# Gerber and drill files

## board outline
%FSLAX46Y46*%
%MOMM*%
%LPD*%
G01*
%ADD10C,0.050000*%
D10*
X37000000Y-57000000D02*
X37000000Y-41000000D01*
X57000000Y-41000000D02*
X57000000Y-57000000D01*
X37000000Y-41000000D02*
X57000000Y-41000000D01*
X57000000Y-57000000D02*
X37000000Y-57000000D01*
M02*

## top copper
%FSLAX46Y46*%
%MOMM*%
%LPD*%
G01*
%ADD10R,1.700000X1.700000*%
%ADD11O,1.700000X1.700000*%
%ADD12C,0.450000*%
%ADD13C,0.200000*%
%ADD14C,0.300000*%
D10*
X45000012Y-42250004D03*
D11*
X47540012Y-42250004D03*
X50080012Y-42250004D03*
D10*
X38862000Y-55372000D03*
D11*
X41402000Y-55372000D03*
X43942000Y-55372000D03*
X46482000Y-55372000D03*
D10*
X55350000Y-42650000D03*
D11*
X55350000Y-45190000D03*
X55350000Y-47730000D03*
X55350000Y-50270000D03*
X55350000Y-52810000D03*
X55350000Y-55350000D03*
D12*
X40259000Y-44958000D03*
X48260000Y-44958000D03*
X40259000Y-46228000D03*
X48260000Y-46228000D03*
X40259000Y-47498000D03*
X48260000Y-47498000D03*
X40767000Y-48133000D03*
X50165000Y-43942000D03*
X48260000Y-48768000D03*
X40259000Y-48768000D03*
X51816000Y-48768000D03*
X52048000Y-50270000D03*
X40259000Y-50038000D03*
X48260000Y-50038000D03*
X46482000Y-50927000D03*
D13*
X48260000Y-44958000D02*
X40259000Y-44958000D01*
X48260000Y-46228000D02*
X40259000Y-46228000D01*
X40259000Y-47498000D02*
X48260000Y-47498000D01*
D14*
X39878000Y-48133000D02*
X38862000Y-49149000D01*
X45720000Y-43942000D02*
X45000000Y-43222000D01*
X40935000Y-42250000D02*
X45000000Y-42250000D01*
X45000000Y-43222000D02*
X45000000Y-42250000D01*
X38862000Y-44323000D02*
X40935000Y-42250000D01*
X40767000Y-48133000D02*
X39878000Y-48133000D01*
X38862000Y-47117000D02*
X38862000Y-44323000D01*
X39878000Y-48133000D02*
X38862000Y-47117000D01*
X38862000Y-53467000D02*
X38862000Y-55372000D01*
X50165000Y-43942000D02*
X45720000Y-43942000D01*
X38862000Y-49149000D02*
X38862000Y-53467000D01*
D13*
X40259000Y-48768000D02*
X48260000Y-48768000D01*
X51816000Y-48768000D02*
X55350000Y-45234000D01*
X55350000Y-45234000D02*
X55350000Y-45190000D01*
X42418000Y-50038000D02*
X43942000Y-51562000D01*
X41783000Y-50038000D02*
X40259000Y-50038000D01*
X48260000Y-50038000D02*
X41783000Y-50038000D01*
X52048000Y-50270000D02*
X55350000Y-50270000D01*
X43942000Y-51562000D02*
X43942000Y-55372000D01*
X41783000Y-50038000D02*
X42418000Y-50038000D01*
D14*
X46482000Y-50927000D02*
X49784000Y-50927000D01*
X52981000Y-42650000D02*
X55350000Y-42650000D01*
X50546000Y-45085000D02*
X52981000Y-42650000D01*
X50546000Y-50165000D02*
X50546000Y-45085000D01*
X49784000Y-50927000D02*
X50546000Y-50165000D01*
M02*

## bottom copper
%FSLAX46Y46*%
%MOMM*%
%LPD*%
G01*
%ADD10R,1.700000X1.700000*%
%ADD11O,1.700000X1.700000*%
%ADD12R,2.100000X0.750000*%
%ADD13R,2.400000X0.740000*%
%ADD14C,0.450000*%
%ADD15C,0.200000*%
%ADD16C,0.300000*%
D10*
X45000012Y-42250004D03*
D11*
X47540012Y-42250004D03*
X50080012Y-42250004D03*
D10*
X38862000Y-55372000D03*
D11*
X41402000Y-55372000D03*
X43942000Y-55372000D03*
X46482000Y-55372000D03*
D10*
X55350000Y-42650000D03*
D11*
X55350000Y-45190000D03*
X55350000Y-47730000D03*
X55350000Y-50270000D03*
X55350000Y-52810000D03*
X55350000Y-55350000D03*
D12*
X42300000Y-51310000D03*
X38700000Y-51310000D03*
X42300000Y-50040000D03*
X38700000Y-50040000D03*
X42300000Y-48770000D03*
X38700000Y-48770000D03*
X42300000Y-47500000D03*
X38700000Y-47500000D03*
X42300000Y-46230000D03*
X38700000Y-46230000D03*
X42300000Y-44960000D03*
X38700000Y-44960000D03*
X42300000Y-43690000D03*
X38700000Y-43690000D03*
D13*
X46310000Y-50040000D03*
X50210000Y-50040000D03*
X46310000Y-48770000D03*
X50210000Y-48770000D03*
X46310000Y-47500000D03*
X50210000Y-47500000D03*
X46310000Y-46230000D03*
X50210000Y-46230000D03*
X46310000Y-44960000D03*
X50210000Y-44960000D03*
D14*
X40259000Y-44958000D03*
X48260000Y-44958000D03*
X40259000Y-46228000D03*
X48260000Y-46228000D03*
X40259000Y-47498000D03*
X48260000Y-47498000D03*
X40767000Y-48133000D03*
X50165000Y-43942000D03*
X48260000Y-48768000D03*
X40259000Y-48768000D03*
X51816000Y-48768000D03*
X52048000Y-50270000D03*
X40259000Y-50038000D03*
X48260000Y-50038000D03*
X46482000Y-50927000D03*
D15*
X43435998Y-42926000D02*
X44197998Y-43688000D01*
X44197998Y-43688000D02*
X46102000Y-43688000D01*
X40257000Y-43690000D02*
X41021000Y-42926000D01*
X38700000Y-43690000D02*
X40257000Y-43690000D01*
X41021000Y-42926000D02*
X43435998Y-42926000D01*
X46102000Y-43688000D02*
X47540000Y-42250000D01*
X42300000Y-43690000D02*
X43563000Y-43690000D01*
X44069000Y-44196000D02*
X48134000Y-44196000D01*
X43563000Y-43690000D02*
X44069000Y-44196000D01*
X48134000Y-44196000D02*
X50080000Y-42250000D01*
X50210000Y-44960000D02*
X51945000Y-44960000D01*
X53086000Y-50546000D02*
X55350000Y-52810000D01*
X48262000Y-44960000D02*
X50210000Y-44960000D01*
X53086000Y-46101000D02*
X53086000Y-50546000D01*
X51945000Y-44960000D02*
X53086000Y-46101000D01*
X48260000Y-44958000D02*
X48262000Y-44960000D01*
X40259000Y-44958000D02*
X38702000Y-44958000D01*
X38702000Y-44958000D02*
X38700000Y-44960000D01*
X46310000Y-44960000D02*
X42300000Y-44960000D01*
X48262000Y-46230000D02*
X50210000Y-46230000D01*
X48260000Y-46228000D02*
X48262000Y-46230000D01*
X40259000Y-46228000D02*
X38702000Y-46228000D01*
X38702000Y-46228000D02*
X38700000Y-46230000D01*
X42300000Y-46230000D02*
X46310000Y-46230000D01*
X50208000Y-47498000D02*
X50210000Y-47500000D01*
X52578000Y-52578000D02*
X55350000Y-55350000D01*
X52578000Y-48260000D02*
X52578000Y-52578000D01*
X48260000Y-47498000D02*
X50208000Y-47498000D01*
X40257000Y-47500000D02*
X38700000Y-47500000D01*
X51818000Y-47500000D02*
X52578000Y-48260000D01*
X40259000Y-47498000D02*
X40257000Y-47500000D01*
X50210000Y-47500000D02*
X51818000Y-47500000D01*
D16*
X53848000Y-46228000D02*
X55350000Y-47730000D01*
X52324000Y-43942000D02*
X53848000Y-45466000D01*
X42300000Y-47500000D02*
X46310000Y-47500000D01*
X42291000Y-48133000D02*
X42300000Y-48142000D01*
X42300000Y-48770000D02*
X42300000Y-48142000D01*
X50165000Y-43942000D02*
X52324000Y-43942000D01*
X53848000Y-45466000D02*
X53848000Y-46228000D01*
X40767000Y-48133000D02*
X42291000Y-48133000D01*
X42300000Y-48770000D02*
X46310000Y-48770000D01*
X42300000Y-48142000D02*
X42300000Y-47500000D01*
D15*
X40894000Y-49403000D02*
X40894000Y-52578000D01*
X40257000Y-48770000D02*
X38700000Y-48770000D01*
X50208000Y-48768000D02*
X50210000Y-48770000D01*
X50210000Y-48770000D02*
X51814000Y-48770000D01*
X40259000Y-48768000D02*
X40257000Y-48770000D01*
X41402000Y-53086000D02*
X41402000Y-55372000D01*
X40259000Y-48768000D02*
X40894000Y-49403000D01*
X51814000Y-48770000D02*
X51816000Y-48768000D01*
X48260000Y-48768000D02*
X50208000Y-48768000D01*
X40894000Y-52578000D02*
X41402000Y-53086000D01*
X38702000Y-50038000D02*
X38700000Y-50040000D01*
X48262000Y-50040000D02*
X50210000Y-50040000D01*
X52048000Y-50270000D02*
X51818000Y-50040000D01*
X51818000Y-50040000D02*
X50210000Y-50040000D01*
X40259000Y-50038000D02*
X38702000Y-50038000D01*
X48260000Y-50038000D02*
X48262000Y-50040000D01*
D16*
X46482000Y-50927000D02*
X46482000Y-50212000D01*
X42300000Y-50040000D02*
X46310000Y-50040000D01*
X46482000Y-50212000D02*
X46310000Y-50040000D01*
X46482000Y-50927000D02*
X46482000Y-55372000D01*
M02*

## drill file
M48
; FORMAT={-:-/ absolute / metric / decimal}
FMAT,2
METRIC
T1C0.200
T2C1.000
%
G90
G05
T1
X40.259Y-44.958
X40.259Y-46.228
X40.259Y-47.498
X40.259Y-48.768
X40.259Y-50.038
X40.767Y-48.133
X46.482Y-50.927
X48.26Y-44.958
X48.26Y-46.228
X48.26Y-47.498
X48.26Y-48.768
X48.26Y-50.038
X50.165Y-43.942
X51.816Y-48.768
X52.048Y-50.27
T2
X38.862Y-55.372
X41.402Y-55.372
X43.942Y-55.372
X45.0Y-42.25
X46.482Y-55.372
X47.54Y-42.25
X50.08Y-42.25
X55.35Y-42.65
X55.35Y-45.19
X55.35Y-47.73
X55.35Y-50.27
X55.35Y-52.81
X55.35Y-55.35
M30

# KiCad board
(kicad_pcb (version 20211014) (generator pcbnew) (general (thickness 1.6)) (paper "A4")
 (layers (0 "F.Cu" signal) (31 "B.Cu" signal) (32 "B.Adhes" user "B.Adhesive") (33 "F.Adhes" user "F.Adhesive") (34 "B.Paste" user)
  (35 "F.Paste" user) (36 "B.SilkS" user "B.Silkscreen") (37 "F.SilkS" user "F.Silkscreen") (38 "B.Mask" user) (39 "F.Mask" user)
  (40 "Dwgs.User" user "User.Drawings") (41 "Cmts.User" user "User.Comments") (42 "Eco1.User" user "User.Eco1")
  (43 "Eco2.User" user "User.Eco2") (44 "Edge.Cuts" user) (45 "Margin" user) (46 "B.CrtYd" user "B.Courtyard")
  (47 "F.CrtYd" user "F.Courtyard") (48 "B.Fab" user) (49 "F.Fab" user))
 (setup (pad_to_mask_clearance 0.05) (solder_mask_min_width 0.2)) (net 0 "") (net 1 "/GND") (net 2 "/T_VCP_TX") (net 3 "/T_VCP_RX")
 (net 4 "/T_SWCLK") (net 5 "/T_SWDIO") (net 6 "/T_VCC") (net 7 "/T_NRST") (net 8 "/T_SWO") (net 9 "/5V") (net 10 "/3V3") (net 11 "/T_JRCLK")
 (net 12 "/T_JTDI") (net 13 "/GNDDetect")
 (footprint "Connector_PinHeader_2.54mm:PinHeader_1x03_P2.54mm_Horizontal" (layer "F.Cu") (at 45.000012 42.250004 90)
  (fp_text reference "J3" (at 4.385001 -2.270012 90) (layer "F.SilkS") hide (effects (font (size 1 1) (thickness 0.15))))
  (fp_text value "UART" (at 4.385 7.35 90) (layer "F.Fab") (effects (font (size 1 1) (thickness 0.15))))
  (pad "1" thru_hole rect locked (at 0 0 90) (size 1.7 1.7) (drill 1) (layers *.Cu *.Mask) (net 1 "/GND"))
  (pad "2" thru_hole oval locked (at 0 2.54 90) (size 1.7 1.7) (drill 1) (layers *.Cu *.Mask) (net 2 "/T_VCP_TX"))
  (pad "3" thru_hole oval locked (at 0 5.08 90) (size 1.7 1.7) (drill 1) (layers *.Cu *.Mask) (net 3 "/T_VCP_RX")))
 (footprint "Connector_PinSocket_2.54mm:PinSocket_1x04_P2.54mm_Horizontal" (layer "F.Cu") (at 38.862 55.372 90)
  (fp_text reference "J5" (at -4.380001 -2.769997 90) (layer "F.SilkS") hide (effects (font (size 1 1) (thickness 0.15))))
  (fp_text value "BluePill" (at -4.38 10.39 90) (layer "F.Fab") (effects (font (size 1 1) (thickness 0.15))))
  (pad "1" thru_hole rect locked (at 0 0 90) (size 1.7 1.7) (drill 1) (layers *.Cu *.Mask) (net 1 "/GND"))
  (pad "2" thru_hole oval locked (at 0 2.54 90) (size 1.7 1.7) (drill 1) (layers *.Cu *.Mask) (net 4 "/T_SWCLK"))
  (pad "3" thru_hole oval locked (at 0 5.08 90) (size 1.7 1.7) (drill 1) (layers *.Cu *.Mask) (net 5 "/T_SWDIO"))
  (pad "4" thru_hole oval locked (at 0 7.62 90) (size 1.7 1.7) (drill 1) (layers *.Cu *.Mask) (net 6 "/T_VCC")))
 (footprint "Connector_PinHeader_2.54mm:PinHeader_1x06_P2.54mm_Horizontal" (layer "F.Cu") (at 55.35 42.65)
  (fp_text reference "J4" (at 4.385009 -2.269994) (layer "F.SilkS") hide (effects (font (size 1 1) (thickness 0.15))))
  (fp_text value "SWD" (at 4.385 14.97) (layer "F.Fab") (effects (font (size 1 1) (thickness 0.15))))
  (pad "1" thru_hole rect locked (at 0 0) (size 1.7 1.7) (drill 1) (layers *.Cu *.Mask) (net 6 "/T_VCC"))
  (pad "2" thru_hole oval locked (at 0 2.54) (size 1.7 1.7) (drill 1) (layers *.Cu *.Mask) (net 4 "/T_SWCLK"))
  (pad "3" thru_hole oval locked (at 0 5.08) (size 1.7 1.7) (drill 1) (layers *.Cu *.Mask) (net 1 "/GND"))
  (pad "4" thru_hole oval locked (at 0 7.62) (size 1.7 1.7) (drill 1) (layers *.Cu *.Mask) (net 5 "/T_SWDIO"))
  (pad "5" thru_hole oval locked (at 0 10.16) (size 1.7 1.7) (drill 1) (layers *.Cu *.Mask) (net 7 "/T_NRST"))
  (pad "6" thru_hole oval locked (at 0 12.7) (size 1.7 1.7) (drill 1) (layers *.Cu *.Mask) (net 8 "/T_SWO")))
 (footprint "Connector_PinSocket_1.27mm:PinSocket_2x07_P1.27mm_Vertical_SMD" (layer "B.Cu") (at 40.5 47.5)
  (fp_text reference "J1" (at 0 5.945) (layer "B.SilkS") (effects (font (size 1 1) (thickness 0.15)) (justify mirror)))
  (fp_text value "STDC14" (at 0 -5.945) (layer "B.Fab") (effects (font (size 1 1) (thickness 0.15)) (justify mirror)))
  (pad "1" smd rect locked (at 1.8 3.81) (size 2.1 0.75) (layers "B.Cu" "B.Paste" "B.Mask") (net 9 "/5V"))
  (pad "2" smd rect locked (at -1.8 3.81) (size 2.1 0.75) (layers "B.Cu" "B.Paste" "B.Mask") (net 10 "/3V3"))
  (pad "3" smd rect locked (at 1.8 2.54) (size 2.1 0.75) (layers "B.Cu" "B.Paste" "B.Mask") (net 6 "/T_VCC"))
  (pad "4" smd rect locked (at -1.8 2.54) (size 2.1 0.75) (layers "B.Cu" "B.Paste" "B.Mask") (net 5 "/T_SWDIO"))
  (pad "5" smd rect locked (at 1.8 1.27) (size 2.1 0.75) (layers "B.Cu" "B.Paste" "B.Mask") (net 1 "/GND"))
  (pad "6" smd rect locked (at -1.8 1.27) (size 2.1 0.75) (layers "B.Cu" "B.Paste" "B.Mask") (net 4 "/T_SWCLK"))
  (pad "7" smd rect locked (at 1.8 0) (size 2.1 0.75) (layers "B.Cu" "B.Paste" "B.Mask") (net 1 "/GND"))
  (pad "8" smd rect locked (at -1.8 0) (size 2.1 0.75) (layers "B.Cu" "B.Paste" "B.Mask") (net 8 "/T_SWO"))
  (pad "9" smd rect locked (at 1.8 -1.27) (size 2.1 0.75) (layers "B.Cu" "B.Paste" "B.Mask") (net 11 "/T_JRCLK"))
  (pad "10" smd rect locked (at -1.8 -1.27) (size 2.1 0.75) (layers "B.Cu" "B.Paste" "B.Mask") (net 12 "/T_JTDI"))
  (pad "11" smd rect locked (at 1.8 -2.54) (size 2.1 0.75) (layers "B.Cu" "B.Paste" "B.Mask") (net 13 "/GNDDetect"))
  (pad "12" smd rect locked (at -1.8 -2.54) (size 2.1 0.75) (layers "B.Cu" "B.Paste" "B.Mask") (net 7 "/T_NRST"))
  (pad "13" smd rect locked (at 1.8 -3.81) (size 2.1 0.75) (layers "B.Cu" "B.Paste" "B.Mask") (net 3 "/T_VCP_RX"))
  (pad "14" smd rect locked (at -1.8 -3.81) (size 2.1 0.75) (layers "B.Cu" "B.Paste" "B.Mask") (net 2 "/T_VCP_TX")))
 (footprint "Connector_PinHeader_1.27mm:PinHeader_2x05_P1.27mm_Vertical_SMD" (layer "B.Cu") (at 48.26 47.5)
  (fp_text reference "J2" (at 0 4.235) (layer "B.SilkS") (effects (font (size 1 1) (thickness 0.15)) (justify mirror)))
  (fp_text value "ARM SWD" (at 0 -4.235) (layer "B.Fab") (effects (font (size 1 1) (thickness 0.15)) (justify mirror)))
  (pad "1" smd rect locked (at -1.95 2.54) (size 2.4 0.74) (layers "B.Cu" "B.Paste" "B.Mask") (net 6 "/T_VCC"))
  (pad "2" smd rect locked (at 1.95 2.54) (size 2.4 0.74) (layers "B.Cu" "B.Paste" "B.Mask") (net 5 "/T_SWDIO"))
  (pad "3" smd rect locked (at -1.95 1.27) (size 2.4 0.74) (layers "B.Cu" "B.Paste" "B.Mask") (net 1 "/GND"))
  (pad "4" smd rect locked (at 1.95 1.27) (size 2.4 0.74) (layers "B.Cu" "B.Paste" "B.Mask") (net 4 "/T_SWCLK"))
  (pad "5" smd rect locked (at -1.95 0) (size 2.4 0.74) (layers "B.Cu" "B.Paste" "B.Mask") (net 1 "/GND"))
  (pad "6" smd rect locked (at 1.95 0) (size 2.4 0.74) (layers "B.Cu" "B.Paste" "B.Mask") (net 8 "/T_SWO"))
  (pad "7" smd rect locked (at -1.95 -1.27) (size 2.4 0.74) (layers "B.Cu" "B.Paste" "B.Mask") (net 11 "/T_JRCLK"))
  (pad "8" smd rect locked (at 1.95 -1.27) (size 2.4 0.74) (layers "B.Cu" "B.Paste" "B.Mask") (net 12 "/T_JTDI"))
  (pad "9" smd rect locked (at -1.95 -2.54) (size 2.4 0.74) (layers "B.Cu" "B.Paste" "B.Mask") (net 13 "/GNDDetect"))
  (pad "10" smd rect locked (at 1.95 -2.54) (size 2.4 0.74) (layers "B.Cu" "B.Paste" "B.Mask") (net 7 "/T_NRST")))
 (gr_line (start 37 57) (end 37 41) (layer "Edge.Cuts") (width 0.05))
 (gr_line (start 57 41) (end 57 57) (layer "Edge.Cuts") (width 0.05))
 (gr_line (start 37 41) (end 57 41) (layer "Edge.Cuts") (width 0.05))
 (gr_line (start 57 57) (end 37 57) (layer "Edge.Cuts") (width 0.05))
 (segment (start 43.435998 42.926) (end 44.197998 43.688) (width 0.2) (layer "B.Cu") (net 2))
 (segment (start 44.197998 43.688) (end 46.102 43.688) (width 0.2) (layer "B.Cu") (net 2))
 (segment (start 40.257 43.69) (end 41.021 42.926) (width 0.2) (layer "B.Cu") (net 2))
 (segment (start 38.7 43.69) (end 40.257 43.69) (width 0.2) (layer "B.Cu") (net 2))
 (segment (start 41.021 42.926) (end 43.435998 42.926) (width 0.2) (layer "B.Cu") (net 2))
 (segment (start 46.102 43.688) (end 47.54 42.25) (width 0.2) (layer "B.Cu") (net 2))
 (segment (start 42.3 43.69) (end 43.563 43.69) (width 0.2) (layer "B.Cu") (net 3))
 (segment (start 44.069 44.196) (end 48.134 44.196) (width 0.2) (layer "B.Cu") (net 3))
 (segment (start 43.563 43.69) (end 44.069 44.196) (width 0.2) (layer "B.Cu") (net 3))
 (segment (start 48.134 44.196) (end 50.08 42.25) (width 0.2) (layer "B.Cu") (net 3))
 (segment (start 48.26 44.958) (end 40.259 44.958) (width 0.2) (layer "F.Cu") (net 7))
 (via (at 40.259 44.958) (size 0.45) (drill 0.2) (layers "F.Cu" "B.Cu") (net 7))
 (via (at 48.26 44.958) (size 0.45) (drill 0.2) (layers "F.Cu" "B.Cu") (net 7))
 (segment (start 50.21 44.96) (end 51.945 44.96) (width 0.2) (layer "B.Cu") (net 7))
 (segment (start 53.086 50.546) (end 55.35 52.81) (width 0.2) (layer "B.Cu") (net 7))
 (segment (start 48.262 44.96) (end 50.21 44.96) (width 0.2) (layer "B.Cu") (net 7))
 (segment (start 53.086 46.101) (end 53.086 50.546) (width 0.2) (layer "B.Cu") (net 7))
 (segment (start 51.945 44.96) (end 53.086 46.101) (width 0.2) (layer "B.Cu") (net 7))
 (segment (start 48.26 44.958) (end 48.262 44.96) (width 0.2) (layer "B.Cu") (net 7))
 (segment (start 40.259 44.958) (end 38.702 44.958) (width 0.2) (layer "B.Cu") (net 7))
 (segment (start 38.702 44.958) (end 38.7 44.96) (width 0.2) (layer "B.Cu") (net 7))
 (segment (start 46.31 44.96) (end 42.3 44.96) (width 0.2) (layer "B.Cu") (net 13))
 (segment (start 48.26 46.228) (end 40.259 46.228) (width 0.2) (layer "F.Cu") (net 12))
 (via (at 40.259 46.228) (size 0.45) (drill 0.2) (layers "F.Cu" "B.Cu") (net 12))
 (via (at 48.26 46.228) (size 0.45) (drill 0.2) (layers "F.Cu" "B.Cu") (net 12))
 (segment (start 48.262 46.23) (end 50.21 46.23) (width 0.2) (layer "B.Cu") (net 12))
 (segment (start 48.26 46.228) (end 48.262 46.23) (width 0.2) (layer "B.Cu") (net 12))
 (segment (start 40.259 46.228) (end 38.702 46.228) (width 0.2) (layer "B.Cu") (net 12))
 (segment (start 38.702 46.228) (end 38.7 46.23) (width 0.2) (layer "B.Cu") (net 12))
 (segment (start 42.3 46.23) (end 46.31 46.23) (width 0.2) (layer "B.Cu") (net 11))
 (segment (start 40.259 47.498) (end 48.26 47.498) (width 0.2) (layer "F.Cu") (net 8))
 (via (at 40.259 47.498) (size 0.45) (drill 0.2) (layers "F.Cu" "B.Cu") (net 8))
 (via (at 48.26 47.498) (size 0.45) (drill 0.2) (layers "F.Cu" "B.Cu") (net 8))
 (segment (start 50.208 47.498) (end 50.21 47.5) (width 0.2) (layer "B.Cu") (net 8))
 (segment (start 52.578 52.578) (end 55.35 55.35) (width 0.2) (layer "B.Cu") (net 8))
 (segment (start 52.578 48.26) (end 52.578 52.578) (width 0.2) (layer "B.Cu") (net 8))
 (segment (start 48.26 47.498) (end 50.208 47.498) (width 0.2) (layer "B.Cu") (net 8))
 (segment (start 40.257 47.5) (end 38.7 47.5) (width 0.2) (layer "B.Cu") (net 8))
 (segment (start 51.818 47.5) (end 52.578 48.26) (width 0.2) (layer "B.Cu") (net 8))
 (segment (start 40.259 47.498) (end 40.257 47.5) (width 0.2) (layer "B.Cu") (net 8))
 (segment (start 50.21 47.5) (end 51.818 47.5) (width 0.2) (layer "B.Cu") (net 8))
 (segment (start 39.878 48.133) (end 38.862 49.149) (width 0.3) (layer "F.Cu") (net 1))
 (segment (start 45.72 43.942) (end 45 43.222) (width 0.3) (layer "F.Cu") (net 1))
 (segment (start 40.935 42.25) (end 45 42.25) (width 0.3) (layer "F.Cu") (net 1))
 (segment (start 45 43.222) (end 45 42.25) (width 0.3) (layer "F.Cu") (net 1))
 (segment (start 38.862 44.323) (end 40.935 42.25) (width 0.3) (layer "F.Cu") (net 1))
 (segment (start 40.767 48.133) (end 39.878 48.133) (width 0.3) (layer "F.Cu") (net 1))
 (segment (start 38.862 47.117) (end 38.862 44.323) (width 0.3) (layer "F.Cu") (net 1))
 (segment (start 39.878 48.133) (end 38.862 47.117) (width 0.3) (layer "F.Cu") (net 1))
 (segment (start 38.862 53.467) (end 38.862 55.372) (width 0.3) (layer "F.Cu") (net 1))
 (segment (start 50.165 43.942) (end 45.72 43.942) (width 0.3) (layer "F.Cu") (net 1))
 (segment (start 38.862 49.149) (end 38.862 53.467) (width 0.3) (layer "F.Cu") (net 1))
 (via (at 40.767 48.133) (size 0.45) (drill 0.2) (layers "F.Cu" "B.Cu") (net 1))
 (via (at 50.165 43.942) (size 0.45) (drill 0.2) (layers "F.Cu" "B.Cu") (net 1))
 (segment (start 53.848 46.228) (end 55.35 47.73) (width 0.3) (layer "B.Cu") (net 1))
 (segment (start 52.324 43.942) (end 53.848 45.466) (width 0.3) (layer "B.Cu") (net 1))
 (segment (start 42.3 47.5) (end 46.31 47.5) (width 0.3) (layer "B.Cu") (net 1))
 (segment (start 42.291 48.133) (end 42.3 48.142) (width 0.3) (layer "B.Cu") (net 1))
 (segment (start 42.3 48.77) (end 42.3 48.142) (width 0.3) (layer "B.Cu") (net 1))
 (segment (start 50.165 43.942) (end 52.324 43.942) (width 0.3) (layer "B.Cu") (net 1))
 (segment (start 53.848 45.466) (end 53.848 46.228) (width 0.3) (layer "B.Cu") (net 1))
 (segment (start 40.767 48.133) (end 42.291 48.133) (width 0.3) (layer "B.Cu") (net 1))
 (segment (start 42.3 48.77) (end 46.31 48.77) (width 0.3) (layer "B.Cu") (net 1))
 (segment (start 42.3 48.142) (end 42.3 47.5) (width 0.3) (layer "B.Cu") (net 1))
 (segment (start 40.259 48.768) (end 48.26 48.768) (width 0.2) (layer "F.Cu") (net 4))
 (segment (start 51.816 48.768) (end 55.35 45.234) (width 0.2) (layer "F.Cu") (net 4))
 (segment (start 55.35 45.234) (end 55.35 45.19) (width 0.2) (layer "F.Cu") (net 4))
 (via (at 48.26 48.768) (size 0.45) (drill 0.2) (layers "F.Cu" "B.Cu") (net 4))
 (via (at 40.259 48.768) (size 0.45) (drill 0.2) (layers "F.Cu" "B.Cu") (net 4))
 (via (at 51.816 48.768) (size 0.45) (drill 0.2) (layers "F.Cu" "B.Cu") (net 4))
 (segment (start 40.894 49.403) (end 40.894 52.578) (width 0.2) (layer "B.Cu") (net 4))
 (segment (start 40.257 48.77) (end 38.7 48.77) (width 0.2) (layer "B.Cu") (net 4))
 (segment (start 50.208 48.768) (end 50.21 48.77) (width 0.2) (layer "B.Cu") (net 4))
 (segment (start 50.21 48.77) (end 51.814 48.77) (width 0.2) (layer "B.Cu") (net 4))
 (segment (start 40.259 48.768) (end 40.257 48.77) (width 0.2) (layer "B.Cu") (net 4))
 (segment (start 41.402 53.086) (end 41.402 55.372) (width 0.2) (layer "B.Cu") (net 4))
 (segment (start 40.259 48.768) (end 40.894 49.403) (width 0.2) (layer "B.Cu") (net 4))
 (segment (start 51.814 48.77) (end 51.816 48.768) (width 0.2) (layer "B.Cu") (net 4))
 (segment (start 48.26 48.768) (end 50.208 48.768) (width 0.2) (layer "B.Cu") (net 4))
 (segment (start 40.894 52.578) (end 41.402 53.086) (width 0.2) (layer "B.Cu") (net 4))
 (segment (start 42.418 50.038) (end 43.942 51.562) (width 0.2) (layer "F.Cu") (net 5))
 (segment (start 41.783 50.038) (end 40.259 50.038) (width 0.2) (layer "F.Cu") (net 5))
 (segment (start 48.26 50.038) (end 41.783 50.038) (width 0.2) (layer "F.Cu") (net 5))
 (segment (start 52.048 50.27) (end 55.35 50.27) (width 0.2) (layer "F.Cu") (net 5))
 (segment (start 43.942 51.562) (end 43.942 55.372) (width 0.2) (layer "F.Cu") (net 5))
 (segment (start 41.783 50.038) (end 42.418 50.038) (width 0.2) (layer "F.Cu") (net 5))
 (via (at 52.048 50.27) (size 0.45) (drill 0.2) (layers "F.Cu" "B.Cu") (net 5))
 (via (at 40.259 50.038) (size 0.45) (drill 0.2) (layers "F.Cu" "B.Cu") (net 5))
 (via (at 48.26 50.038) (size 0.45) (drill 0.2) (layers "F.Cu" "B.Cu") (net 5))
 (segment (start 38.702 50.038) (end 38.7 50.04) (width 0.2) (layer "B.Cu") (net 5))
 (segment (start 48.262 50.04) (end 50.21 50.04) (width 0.2) (layer "B.Cu") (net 5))
 (segment (start 52.048 50.27) (end 51.818 50.04) (width 0.2) (layer "B.Cu") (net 5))
 (segment (start 51.818 50.04) (end 50.21 50.04) (width 0.2) (layer "B.Cu") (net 5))
 (segment (start 40.259 50.038) (end 38.702 50.038) (width 0.2) (layer "B.Cu") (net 5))
 (segment (start 48.26 50.038) (end 48.262 50.04) (width 0.2) (layer "B.Cu") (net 5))
 (segment (start 46.482 50.927) (end 49.784 50.927) (width 0.3) (layer "F.Cu") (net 6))
 (segment (start 52.981 42.65) (end 55.35 42.65) (width 0.3) (layer "F.Cu") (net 6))
 (segment (start 50.546 45.085) (end 52.981 42.65) (width 0.3) (layer "F.Cu") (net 6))
 (segment (start 50.546 50.165) (end 50.546 45.085) (width 0.3) (layer "F.Cu") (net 6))
 (segment (start 49.784 50.927) (end 50.546 50.165) (width 0.3) (layer "F.Cu") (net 6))
 (via (at 46.482 50.927) (size 0.45) (drill 0.2) (layers "F.Cu" "B.Cu") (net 6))
 (segment (start 46.482 50.927) (end 46.482 50.212) (width 0.3) (layer "B.Cu") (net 6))
 (segment (start 42.3 50.04) (end 46.31 50.04) (width 0.3) (layer "B.Cu") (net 6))
 (segment (start 46.482 50.212) (end 46.31 50.04) (width 0.3) (layer "B.Cu") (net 6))
 (segment (start 46.482 50.927) (end 46.482 55.372) (width 0.3) (layer "B.Cu") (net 6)))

